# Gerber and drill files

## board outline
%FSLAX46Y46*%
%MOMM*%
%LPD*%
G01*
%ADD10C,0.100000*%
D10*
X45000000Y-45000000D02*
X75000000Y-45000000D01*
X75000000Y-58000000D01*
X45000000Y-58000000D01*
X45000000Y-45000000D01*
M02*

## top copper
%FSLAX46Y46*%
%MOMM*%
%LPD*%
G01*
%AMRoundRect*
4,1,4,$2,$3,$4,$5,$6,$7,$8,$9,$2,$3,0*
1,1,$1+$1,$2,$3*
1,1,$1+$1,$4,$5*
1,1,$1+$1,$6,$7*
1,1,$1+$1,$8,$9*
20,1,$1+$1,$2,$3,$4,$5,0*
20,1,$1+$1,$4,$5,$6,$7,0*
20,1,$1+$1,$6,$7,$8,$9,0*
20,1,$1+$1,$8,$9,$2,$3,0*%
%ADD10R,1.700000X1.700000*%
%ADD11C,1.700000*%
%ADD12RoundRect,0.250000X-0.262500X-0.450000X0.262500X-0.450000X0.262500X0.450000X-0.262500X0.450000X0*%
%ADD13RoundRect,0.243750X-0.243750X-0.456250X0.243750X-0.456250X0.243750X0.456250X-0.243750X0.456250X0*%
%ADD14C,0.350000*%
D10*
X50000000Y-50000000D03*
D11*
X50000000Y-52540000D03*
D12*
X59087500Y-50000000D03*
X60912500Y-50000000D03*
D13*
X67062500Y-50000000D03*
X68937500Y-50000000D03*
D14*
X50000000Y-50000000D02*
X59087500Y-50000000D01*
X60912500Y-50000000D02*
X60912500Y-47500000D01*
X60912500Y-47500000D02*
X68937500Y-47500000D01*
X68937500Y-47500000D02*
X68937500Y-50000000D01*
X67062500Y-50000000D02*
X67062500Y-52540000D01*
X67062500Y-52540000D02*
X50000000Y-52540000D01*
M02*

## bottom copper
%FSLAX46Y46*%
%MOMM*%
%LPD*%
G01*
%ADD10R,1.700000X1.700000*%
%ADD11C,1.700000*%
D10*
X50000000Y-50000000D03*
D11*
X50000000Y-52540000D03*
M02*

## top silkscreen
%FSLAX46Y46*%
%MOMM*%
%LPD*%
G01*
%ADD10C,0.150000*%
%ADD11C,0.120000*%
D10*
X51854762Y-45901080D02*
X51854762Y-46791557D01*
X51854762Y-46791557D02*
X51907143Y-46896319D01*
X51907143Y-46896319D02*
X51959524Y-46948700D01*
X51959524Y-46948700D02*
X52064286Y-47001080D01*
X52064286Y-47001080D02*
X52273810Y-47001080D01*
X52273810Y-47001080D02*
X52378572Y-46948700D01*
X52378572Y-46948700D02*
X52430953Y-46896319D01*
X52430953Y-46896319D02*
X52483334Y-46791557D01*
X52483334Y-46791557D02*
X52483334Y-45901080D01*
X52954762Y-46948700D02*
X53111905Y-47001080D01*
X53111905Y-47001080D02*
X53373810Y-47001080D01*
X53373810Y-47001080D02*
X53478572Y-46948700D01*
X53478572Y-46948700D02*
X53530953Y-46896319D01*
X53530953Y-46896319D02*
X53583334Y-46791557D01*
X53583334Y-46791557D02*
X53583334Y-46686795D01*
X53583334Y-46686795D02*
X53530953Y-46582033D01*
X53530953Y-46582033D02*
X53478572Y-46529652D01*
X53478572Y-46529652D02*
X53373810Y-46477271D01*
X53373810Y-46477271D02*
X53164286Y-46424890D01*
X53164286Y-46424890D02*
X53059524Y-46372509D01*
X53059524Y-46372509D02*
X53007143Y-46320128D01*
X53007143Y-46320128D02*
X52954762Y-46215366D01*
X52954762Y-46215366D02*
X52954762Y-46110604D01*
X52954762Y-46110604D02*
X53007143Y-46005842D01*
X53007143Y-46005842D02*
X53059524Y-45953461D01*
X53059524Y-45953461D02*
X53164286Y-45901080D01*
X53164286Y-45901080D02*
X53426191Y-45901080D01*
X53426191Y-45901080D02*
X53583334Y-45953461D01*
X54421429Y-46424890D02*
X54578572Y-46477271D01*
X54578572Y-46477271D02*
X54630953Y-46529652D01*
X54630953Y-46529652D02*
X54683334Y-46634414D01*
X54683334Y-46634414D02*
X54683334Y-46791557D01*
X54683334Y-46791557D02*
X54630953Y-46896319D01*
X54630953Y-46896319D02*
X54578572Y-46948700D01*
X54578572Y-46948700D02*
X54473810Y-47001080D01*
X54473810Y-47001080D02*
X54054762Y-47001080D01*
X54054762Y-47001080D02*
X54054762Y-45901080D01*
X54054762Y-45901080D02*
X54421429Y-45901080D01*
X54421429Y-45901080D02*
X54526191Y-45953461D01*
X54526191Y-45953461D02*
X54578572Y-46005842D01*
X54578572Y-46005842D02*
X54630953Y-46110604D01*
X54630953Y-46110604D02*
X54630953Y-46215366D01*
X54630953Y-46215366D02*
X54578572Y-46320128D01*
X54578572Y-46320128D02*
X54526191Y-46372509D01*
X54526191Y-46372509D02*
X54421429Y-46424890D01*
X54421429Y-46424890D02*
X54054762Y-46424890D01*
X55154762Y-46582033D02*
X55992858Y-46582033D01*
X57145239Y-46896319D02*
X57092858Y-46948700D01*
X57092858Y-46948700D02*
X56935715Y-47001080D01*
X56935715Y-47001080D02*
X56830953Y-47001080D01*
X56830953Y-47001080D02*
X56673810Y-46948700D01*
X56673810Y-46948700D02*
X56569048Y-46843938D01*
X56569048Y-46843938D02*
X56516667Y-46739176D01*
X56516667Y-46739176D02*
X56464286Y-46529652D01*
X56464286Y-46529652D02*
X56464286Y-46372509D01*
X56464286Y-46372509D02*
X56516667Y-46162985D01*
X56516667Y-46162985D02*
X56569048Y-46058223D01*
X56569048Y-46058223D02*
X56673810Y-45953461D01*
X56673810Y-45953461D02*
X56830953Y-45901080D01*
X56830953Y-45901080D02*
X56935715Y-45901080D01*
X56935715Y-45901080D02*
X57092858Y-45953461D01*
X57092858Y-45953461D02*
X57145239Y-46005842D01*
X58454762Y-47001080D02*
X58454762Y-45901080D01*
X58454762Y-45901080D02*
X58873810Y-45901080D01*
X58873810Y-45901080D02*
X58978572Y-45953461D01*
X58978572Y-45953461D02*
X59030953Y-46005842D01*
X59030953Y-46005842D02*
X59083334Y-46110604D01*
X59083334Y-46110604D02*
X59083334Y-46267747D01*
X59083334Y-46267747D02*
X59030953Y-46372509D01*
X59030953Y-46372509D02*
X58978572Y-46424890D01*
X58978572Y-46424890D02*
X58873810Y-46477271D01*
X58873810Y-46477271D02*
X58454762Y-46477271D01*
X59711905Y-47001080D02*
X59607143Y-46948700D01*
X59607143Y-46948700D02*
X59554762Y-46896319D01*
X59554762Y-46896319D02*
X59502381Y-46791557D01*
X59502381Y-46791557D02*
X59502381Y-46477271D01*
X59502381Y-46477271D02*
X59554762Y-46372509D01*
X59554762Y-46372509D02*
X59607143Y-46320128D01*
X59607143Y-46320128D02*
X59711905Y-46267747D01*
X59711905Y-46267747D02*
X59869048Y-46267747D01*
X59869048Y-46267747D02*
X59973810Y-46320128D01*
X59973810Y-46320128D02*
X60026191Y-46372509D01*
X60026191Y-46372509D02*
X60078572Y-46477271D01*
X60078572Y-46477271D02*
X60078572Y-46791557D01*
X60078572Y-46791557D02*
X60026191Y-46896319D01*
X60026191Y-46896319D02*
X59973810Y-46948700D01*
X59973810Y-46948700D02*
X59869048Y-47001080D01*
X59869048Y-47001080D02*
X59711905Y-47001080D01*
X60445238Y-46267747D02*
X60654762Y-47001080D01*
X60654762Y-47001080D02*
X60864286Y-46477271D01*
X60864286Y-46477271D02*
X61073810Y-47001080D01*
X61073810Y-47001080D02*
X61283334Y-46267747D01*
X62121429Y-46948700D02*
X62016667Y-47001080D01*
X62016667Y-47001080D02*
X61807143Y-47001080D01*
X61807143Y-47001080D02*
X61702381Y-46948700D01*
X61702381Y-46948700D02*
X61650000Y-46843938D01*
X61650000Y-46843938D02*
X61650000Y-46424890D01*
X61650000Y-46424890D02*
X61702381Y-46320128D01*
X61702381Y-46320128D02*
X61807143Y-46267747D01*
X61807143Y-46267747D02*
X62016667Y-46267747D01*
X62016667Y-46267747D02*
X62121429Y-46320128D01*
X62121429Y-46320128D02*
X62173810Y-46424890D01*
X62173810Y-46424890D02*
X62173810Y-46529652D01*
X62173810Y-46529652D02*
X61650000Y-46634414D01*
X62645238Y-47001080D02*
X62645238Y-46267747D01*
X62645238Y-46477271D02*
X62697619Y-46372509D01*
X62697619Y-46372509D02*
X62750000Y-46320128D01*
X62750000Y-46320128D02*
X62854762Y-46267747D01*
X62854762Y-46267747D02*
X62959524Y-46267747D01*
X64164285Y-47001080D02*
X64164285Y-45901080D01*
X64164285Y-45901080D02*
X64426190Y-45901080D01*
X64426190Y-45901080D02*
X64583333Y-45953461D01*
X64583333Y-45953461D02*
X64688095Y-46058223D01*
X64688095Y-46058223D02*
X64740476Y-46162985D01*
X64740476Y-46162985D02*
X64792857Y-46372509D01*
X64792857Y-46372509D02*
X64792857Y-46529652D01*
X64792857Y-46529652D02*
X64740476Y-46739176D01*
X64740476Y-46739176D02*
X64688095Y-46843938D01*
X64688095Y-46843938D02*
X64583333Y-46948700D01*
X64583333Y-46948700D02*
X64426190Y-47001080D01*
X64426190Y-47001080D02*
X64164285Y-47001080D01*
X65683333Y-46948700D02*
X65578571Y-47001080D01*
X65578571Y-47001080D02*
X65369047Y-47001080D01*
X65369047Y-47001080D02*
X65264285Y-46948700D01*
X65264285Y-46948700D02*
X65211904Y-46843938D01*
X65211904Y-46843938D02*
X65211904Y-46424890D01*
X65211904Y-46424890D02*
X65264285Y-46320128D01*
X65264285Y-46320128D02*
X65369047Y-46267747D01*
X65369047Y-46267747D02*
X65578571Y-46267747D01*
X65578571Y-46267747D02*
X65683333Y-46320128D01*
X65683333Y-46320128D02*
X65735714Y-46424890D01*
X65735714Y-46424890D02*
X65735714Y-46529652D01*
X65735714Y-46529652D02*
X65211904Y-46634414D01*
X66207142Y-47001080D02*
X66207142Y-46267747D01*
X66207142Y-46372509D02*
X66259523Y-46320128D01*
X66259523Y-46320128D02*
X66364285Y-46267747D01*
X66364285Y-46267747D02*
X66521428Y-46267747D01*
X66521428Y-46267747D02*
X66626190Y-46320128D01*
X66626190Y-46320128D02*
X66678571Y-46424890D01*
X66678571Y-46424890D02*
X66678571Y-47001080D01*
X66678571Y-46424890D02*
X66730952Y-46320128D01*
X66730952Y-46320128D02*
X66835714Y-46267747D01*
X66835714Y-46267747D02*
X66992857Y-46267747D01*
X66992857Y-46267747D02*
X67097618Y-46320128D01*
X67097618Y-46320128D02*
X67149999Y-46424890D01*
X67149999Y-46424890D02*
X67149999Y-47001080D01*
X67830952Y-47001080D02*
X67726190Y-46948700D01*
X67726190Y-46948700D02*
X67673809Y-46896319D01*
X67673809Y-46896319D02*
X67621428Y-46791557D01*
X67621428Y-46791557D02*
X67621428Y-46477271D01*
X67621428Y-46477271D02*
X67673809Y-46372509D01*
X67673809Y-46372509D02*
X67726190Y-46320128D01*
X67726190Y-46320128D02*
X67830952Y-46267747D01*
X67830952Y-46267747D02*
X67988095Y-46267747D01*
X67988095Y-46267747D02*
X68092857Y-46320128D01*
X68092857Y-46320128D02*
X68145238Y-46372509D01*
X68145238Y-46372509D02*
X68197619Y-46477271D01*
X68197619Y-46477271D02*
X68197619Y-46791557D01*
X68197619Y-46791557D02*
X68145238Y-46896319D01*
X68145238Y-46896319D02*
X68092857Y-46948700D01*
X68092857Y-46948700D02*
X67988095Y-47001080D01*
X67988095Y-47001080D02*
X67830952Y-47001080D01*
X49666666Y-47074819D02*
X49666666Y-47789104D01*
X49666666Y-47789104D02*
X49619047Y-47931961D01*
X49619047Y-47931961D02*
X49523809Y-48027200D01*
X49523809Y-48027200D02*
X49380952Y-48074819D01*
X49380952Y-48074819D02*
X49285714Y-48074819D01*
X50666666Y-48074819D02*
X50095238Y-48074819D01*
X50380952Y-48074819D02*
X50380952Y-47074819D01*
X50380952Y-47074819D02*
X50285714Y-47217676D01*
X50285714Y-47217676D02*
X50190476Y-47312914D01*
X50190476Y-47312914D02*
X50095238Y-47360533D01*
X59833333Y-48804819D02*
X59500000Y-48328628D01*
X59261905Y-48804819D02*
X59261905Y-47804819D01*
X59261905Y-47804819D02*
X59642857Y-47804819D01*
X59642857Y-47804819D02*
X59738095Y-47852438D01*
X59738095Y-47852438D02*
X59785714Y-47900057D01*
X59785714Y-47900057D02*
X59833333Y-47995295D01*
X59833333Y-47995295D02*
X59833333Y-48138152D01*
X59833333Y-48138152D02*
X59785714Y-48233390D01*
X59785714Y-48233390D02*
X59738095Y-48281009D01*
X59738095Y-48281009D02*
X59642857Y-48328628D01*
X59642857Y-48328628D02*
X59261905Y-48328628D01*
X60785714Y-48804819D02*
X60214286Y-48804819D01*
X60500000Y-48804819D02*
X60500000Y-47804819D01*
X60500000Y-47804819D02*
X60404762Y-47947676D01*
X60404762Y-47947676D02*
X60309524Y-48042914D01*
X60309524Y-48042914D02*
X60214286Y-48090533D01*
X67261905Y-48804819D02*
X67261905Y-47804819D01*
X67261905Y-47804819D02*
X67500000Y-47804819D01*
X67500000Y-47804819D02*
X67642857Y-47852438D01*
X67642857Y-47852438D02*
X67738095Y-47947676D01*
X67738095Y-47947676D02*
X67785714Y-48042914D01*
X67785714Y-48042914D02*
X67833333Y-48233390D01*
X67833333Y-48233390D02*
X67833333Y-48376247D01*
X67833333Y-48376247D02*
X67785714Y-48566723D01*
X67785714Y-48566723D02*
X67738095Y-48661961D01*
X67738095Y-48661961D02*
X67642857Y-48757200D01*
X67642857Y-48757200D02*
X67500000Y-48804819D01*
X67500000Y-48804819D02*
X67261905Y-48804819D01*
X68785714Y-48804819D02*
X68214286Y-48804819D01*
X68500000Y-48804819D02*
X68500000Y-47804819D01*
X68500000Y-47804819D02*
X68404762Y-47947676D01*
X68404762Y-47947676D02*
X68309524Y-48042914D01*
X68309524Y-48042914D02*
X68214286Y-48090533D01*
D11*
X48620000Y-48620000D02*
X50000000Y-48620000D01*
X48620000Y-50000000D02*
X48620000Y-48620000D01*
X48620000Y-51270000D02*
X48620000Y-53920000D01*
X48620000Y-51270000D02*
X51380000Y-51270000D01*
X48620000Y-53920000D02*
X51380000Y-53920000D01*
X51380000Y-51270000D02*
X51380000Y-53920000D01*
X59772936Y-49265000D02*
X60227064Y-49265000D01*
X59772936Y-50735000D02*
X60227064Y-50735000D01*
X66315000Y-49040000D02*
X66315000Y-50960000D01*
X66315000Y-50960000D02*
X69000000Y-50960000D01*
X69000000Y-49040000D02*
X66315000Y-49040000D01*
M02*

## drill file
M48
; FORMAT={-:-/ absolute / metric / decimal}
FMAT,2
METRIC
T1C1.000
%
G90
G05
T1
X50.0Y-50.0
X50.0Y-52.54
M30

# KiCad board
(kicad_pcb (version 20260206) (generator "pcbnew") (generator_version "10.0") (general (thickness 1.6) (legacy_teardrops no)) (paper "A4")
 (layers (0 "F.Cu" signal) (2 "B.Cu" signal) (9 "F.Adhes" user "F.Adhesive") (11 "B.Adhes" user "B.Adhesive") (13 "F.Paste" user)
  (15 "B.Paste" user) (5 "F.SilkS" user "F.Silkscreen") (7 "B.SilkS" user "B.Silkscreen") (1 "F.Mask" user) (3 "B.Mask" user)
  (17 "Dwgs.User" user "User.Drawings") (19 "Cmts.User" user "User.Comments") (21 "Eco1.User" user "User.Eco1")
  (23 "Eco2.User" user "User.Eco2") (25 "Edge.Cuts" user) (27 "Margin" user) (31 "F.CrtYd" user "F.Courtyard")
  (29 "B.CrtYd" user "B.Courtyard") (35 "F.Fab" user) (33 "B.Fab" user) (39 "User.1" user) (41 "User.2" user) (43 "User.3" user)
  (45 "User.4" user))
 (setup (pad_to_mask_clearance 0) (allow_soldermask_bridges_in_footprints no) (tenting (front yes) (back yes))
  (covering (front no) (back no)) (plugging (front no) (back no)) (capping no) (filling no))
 (gr_rect (start 45 45) (end 75 58) (stroke (width 0.1) (type solid)) (fill no) (layer "Edge.Cuts"))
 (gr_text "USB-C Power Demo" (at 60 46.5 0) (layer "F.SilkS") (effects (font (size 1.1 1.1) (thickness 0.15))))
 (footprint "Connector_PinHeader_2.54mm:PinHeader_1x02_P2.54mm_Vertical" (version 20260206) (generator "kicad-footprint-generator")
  (layer "F.Cu") (at 50 50 0)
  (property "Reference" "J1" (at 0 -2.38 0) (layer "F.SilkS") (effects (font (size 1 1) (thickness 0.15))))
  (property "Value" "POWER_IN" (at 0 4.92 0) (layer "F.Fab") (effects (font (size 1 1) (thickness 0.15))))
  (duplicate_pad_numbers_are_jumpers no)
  (fp_line (start -1.38 -1.38) (end 0 -1.38) (stroke (width 0.12) (type solid)) (layer "F.SilkS"))
  (fp_line (start -1.38 0) (end -1.38 -1.38) (stroke (width 0.12) (type solid)) (layer "F.SilkS"))
  (fp_line (start -1.38 1.27) (end -1.38 3.92) (stroke (width 0.12) (type solid)) (layer "F.SilkS"))
  (fp_line (start -1.38 1.27) (end 1.38 1.27) (stroke (width 0.12) (type solid)) (layer "F.SilkS"))
  (fp_line (start -1.38 3.92) (end 1.38 3.92) (stroke (width 0.12) (type solid)) (layer "F.SilkS"))
  (fp_line (start 1.38 1.27) (end 1.38 3.92) (stroke (width 0.12) (type solid)) (layer "F.SilkS"))
  (pad "1" thru_hole rect (at 0 0) (size 1.7 1.7) (drill 1) (layers "*.Cu" "*.Mask") (remove_unused_layers no) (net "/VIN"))
  (pad "2" thru_hole circle (at 0 2.54) (size 1.7 1.7) (drill 1) (layers "*.Cu" "*.Mask") (remove_unused_layers no) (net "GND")))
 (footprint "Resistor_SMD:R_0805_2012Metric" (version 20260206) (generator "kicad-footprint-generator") (layer "F.Cu") (at 60 50 0)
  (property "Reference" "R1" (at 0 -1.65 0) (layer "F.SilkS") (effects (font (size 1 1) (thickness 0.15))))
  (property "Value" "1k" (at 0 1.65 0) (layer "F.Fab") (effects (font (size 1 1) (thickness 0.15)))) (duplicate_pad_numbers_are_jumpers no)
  (fp_line (start -0.227064 -0.735) (end 0.227064 -0.735) (stroke (width 0.12) (type solid)) (layer "F.SilkS"))
  (fp_line (start -0.227064 0.735) (end 0.227064 0.735) (stroke (width 0.12) (type solid)) (layer "F.SilkS"))
  (pad "1" smd roundrect (at -0.9125 0) (size 1.025 1.4) (layers "F.Cu" "F.Mask" "F.Paste") (roundrect_rratio 0.243902) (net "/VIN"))
  (pad "2" smd roundrect (at 0.9125 0) (size 1.025 1.4) (layers "F.Cu" "F.Mask" "F.Paste") (roundrect_rratio 0.243902) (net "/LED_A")))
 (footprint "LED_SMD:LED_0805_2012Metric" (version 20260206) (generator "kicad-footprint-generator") (layer "F.Cu") (at 68 50 0)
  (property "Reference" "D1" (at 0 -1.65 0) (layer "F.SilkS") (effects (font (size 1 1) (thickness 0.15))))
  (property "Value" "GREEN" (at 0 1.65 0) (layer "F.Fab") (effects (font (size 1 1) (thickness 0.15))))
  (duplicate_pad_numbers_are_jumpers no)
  (fp_line (start -1.685 -0.96) (end -1.685 0.96) (stroke (width 0.12) (type solid)) (layer "F.SilkS"))
  (fp_line (start -1.685 0.96) (end 1 0.96) (stroke (width 0.12) (type solid)) (layer "F.SilkS"))
  (fp_line (start 1 -0.96) (end -1.685 -0.96) (stroke (width 0.12) (type solid)) (layer "F.SilkS"))
  (pad "1" smd roundrect (at -0.9375 0) (size 0.975 1.4) (layers "F.Cu" "F.Mask" "F.Paste") (roundrect_rratio 0.25) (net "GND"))
  (pad "2" smd roundrect (at 0.9375 0) (size 0.975 1.4) (layers "F.Cu" "F.Mask" "F.Paste") (roundrect_rratio 0.25) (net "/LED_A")))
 (segment (start 50 50) (end 59.0875 50) (width 0.35) (layer "F.Cu") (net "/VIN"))
 (segment (start 60.9125 50) (end 60.9125 47.5) (width 0.35) (layer "F.Cu") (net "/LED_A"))
 (segment (start 60.9125 47.5) (end 68.9375 47.5) (width 0.35) (layer "F.Cu") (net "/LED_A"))
 (segment (start 68.9375 47.5) (end 68.9375 50) (width 0.35) (layer "F.Cu") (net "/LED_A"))
 (segment (start 67.0625 50) (end 67.0625 52.54) (width 0.35) (layer "F.Cu") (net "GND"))
 (segment (start 67.0625 52.54) (end 50 52.54) (width 0.35) (layer "F.Cu") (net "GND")))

